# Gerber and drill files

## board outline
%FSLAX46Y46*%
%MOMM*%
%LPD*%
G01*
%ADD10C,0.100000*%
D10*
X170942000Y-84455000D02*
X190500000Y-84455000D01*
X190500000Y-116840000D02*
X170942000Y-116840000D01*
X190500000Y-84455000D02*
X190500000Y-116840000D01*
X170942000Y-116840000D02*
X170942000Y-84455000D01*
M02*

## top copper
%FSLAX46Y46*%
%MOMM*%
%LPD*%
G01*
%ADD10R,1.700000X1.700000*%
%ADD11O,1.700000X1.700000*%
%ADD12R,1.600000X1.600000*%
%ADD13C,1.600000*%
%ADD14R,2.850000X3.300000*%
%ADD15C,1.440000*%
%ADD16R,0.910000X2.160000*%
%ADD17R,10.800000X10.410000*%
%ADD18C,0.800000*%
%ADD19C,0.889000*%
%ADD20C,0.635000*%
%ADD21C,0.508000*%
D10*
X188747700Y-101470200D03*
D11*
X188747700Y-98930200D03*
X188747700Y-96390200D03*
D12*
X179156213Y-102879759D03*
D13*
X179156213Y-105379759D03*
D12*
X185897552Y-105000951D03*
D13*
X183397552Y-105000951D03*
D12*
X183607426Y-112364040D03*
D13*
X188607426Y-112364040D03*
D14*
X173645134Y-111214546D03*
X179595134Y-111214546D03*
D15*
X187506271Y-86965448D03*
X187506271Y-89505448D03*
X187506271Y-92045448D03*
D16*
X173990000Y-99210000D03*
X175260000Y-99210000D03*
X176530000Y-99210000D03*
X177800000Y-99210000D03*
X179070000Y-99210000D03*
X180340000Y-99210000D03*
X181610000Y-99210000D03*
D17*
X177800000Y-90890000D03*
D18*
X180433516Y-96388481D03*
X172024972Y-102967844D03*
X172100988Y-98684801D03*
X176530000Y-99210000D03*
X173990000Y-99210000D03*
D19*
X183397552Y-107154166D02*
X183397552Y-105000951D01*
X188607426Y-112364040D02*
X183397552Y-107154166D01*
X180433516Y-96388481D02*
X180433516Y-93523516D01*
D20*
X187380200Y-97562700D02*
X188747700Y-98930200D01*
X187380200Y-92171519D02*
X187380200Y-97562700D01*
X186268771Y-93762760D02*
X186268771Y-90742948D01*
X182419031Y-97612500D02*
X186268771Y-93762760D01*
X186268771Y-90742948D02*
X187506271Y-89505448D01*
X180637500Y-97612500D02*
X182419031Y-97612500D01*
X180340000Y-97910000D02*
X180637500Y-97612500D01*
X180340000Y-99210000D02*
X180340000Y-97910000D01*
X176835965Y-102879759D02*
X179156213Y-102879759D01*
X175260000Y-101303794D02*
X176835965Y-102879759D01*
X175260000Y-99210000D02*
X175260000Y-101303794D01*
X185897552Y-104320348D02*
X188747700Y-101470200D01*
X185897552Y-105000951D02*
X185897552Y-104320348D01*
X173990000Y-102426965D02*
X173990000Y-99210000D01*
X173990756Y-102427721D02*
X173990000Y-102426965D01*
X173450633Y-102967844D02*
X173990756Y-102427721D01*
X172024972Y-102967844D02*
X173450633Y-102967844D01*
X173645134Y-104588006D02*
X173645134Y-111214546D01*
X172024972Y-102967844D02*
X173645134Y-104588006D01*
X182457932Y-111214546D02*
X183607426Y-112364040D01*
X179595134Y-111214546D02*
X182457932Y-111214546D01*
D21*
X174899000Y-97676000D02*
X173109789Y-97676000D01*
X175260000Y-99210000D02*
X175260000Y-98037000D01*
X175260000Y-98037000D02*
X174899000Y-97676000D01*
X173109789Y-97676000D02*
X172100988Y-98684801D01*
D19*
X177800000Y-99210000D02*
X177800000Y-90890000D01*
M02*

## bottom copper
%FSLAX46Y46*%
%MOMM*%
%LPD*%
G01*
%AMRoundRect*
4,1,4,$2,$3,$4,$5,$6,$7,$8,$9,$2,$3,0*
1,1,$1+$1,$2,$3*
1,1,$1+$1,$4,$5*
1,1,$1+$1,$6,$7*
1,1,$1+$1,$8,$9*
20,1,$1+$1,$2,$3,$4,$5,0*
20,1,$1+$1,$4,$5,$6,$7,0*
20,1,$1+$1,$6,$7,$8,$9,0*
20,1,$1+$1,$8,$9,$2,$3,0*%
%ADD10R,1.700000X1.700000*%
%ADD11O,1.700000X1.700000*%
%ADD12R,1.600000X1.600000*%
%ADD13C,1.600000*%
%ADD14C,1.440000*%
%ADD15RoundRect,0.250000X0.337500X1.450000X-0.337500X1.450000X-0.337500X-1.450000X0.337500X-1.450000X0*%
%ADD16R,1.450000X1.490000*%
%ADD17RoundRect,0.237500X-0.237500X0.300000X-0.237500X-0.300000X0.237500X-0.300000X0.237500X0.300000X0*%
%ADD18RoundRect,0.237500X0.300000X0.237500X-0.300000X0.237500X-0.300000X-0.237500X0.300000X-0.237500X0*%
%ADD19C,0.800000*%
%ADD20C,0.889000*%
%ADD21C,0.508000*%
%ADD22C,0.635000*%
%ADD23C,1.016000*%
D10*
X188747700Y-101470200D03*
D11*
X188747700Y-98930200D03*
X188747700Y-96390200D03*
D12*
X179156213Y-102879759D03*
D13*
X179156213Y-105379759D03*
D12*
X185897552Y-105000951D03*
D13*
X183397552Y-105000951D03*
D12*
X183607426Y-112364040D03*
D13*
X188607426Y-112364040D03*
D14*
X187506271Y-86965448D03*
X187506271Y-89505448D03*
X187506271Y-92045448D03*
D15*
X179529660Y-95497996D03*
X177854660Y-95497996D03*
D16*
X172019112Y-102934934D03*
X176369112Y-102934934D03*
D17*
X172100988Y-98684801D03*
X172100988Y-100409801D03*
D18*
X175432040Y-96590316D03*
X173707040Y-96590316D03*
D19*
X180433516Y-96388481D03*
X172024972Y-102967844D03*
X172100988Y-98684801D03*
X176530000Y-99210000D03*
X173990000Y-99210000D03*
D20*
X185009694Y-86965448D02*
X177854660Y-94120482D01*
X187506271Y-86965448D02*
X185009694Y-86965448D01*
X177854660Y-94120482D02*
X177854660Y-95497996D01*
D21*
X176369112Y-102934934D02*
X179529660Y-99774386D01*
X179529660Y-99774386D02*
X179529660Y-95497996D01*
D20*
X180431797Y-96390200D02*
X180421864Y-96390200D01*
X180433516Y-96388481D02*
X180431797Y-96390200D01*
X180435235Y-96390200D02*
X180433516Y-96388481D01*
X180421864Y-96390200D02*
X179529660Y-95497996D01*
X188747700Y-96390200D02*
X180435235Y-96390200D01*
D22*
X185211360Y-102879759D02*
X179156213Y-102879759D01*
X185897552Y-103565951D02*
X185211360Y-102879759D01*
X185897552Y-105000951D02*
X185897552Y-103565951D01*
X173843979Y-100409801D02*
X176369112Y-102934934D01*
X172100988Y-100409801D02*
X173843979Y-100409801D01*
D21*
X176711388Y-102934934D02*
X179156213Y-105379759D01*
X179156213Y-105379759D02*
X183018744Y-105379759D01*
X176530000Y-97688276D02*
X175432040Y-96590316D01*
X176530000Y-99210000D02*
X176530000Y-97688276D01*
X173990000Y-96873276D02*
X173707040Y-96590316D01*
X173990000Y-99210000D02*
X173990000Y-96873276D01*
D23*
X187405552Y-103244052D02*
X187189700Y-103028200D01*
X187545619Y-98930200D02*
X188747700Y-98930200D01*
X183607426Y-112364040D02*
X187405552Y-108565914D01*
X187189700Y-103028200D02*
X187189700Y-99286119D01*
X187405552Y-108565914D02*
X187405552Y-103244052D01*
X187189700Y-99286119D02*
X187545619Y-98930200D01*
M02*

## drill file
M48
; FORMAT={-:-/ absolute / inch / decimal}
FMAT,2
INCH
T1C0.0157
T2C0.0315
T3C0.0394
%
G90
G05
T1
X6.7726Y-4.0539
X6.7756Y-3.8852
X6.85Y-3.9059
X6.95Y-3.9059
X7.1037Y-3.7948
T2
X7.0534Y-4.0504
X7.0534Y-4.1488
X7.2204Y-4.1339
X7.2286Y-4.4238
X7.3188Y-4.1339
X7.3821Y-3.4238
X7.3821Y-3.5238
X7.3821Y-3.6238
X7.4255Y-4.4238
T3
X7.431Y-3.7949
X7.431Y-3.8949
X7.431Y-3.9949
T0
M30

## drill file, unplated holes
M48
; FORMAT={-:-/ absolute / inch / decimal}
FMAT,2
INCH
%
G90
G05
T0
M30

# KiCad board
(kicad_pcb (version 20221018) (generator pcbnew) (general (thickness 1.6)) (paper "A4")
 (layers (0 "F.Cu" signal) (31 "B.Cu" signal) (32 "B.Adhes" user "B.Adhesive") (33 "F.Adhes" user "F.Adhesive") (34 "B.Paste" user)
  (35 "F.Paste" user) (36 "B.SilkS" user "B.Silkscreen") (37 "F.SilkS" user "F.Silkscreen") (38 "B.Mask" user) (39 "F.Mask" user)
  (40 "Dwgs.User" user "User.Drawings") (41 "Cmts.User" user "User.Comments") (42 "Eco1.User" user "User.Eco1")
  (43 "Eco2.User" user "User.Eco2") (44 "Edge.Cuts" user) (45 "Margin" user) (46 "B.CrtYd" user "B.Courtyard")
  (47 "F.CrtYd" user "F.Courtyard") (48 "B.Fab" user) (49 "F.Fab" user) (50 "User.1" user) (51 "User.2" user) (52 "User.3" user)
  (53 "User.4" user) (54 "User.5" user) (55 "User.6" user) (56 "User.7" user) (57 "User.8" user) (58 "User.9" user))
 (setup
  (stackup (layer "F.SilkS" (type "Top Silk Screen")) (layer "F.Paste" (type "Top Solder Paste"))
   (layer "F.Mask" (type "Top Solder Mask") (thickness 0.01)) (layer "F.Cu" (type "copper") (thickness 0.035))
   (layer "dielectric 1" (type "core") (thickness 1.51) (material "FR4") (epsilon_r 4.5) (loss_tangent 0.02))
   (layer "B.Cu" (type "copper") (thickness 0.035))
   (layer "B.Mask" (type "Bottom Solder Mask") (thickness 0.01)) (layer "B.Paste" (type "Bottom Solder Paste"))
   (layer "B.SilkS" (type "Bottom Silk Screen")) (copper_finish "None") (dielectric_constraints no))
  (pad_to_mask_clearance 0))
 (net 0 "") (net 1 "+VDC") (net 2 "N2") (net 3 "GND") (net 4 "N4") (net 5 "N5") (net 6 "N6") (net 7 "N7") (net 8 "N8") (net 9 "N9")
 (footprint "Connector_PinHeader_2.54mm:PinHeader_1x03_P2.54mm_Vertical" (layer "F.Cu") (at 188.7477 101.4702 180)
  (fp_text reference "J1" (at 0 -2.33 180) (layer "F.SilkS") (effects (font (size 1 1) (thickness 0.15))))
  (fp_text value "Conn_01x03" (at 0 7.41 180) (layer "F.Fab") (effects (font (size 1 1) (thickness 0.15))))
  (pad "1" thru_hole rect (at 0 0 180) (size 1.7 1.7) (drill 1) (layers "*.Cu" "*.Mask") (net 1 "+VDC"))
  (pad "2" thru_hole oval (at 0 2.54 180) (size 1.7 1.7) (drill 1) (layers "*.Cu" "*.Mask") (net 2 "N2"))
  (pad "3" thru_hole oval (at 0 5.08 180) (size 1.7 1.7) (drill 1) (layers "*.Cu" "*.Mask") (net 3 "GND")))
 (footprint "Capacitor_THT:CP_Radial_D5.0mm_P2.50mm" (layer "F.Cu") (at 179.156213 102.879759 -90)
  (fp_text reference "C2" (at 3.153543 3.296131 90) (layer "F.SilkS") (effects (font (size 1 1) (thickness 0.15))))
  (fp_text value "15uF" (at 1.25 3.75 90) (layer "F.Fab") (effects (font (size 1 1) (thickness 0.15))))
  (pad "1" thru_hole rect (at 0 0 270) (size 1.6 1.6) (drill 0.8) (layers "*.Cu" "*.Mask") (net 1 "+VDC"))
  (pad "2" thru_hole circle (at 2.5 0 270) (size 1.6 1.6) (drill 0.8) (layers "*.Cu" "*.Mask") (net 3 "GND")))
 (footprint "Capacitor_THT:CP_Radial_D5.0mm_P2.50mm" (layer "F.Cu") (at 185.897552 105.000951 180)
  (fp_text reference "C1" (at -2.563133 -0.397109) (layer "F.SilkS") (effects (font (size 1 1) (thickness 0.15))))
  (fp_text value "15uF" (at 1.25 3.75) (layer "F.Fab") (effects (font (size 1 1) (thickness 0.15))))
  (pad "1" thru_hole rect (at 0 0 180) (size 1.6 1.6) (drill 0.8) (layers "*.Cu" "*.Mask") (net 1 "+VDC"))
  (pad "2" thru_hole circle (at 2.5 0 180) (size 1.6 1.6) (drill 0.8) (layers "*.Cu" "*.Mask") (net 3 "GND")))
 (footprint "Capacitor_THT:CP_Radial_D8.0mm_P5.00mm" (layer "F.Cu") (at 183.607426 112.36404)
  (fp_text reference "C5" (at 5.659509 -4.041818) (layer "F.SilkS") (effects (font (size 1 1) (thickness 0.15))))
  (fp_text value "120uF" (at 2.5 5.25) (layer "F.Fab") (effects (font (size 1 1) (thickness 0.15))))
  (pad "1" thru_hole rect (at 0 0) (size 1.6 1.6) (drill 0.8) (layers "*.Cu" "*.Mask") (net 2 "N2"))
  (pad "2" thru_hole circle (at 5 0) (size 1.6 1.6) (drill 0.8) (layers "*.Cu" "*.Mask") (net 3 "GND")))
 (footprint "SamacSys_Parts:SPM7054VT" (layer "F.Cu") (at 176.620134 111.214546)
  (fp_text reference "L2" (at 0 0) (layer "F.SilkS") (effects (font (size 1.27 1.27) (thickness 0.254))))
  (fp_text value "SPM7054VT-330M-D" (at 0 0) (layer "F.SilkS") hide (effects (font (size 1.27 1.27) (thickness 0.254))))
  (pad "1" smd rect (at -2.975 0) (size 2.85 3.3) (layers "F.Cu" "F.Paste" "F.Mask") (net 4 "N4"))
  (pad "2" smd rect (at 2.975 0) (size 2.85 3.3) (layers "F.Cu" "F.Paste" "F.Mask") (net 2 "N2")))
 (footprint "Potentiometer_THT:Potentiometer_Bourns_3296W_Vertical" (layer "F.Cu") (at 187.506271 86.965448 90)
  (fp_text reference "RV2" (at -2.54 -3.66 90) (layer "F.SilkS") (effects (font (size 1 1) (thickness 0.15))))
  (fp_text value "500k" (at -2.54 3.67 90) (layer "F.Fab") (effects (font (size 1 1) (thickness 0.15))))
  (pad "1" thru_hole circle (at 0 0 90) (size 1.44 1.44) (drill 0.8) (layers "*.Cu" "*.Mask") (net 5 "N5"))
  (pad "2" thru_hole circle (at -2.54 0 90) (size 1.44 1.44) (drill 0.8) (layers "*.Cu" "*.Mask") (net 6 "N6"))
  (pad "3" thru_hole circle (at -5.08 0 90) (size 1.44 1.44) (drill 0.8) (layers "*.Cu" "*.Mask") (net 2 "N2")))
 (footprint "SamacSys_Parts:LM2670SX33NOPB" (layer "F.Cu") (at 177.8 91.44 -90)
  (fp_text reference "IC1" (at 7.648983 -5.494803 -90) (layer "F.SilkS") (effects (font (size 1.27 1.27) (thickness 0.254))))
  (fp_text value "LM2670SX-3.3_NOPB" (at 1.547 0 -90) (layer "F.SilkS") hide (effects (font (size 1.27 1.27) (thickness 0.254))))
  (pad "1" smd rect (at 7.77 3.81) (size 0.91 2.16) (layers "F.Cu" "F.Paste" "F.Mask") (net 4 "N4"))
  (pad "2" smd rect (at 7.77 2.54) (size 0.91 2.16) (layers "F.Cu" "F.Paste" "F.Mask") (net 1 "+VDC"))
  (pad "3" smd rect (at 7.77 1.27) (size 0.91 2.16) (layers "F.Cu" "F.Paste" "F.Mask") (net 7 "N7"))
  (pad "4" smd rect (at 7.77 0) (size 0.91 2.16) (layers "F.Cu" "F.Paste" "F.Mask") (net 3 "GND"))
  (pad "5" smd rect (at 7.77 -1.27) (size 0.91 2.16) (layers "F.Cu" "F.Paste" "F.Mask") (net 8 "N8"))
  (pad "6" smd rect (at 7.77 -2.54) (size 0.91 2.16) (layers "F.Cu" "F.Paste" "F.Mask") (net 6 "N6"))
  (pad "7" smd rect (at 7.77 -3.81) (size 0.91 2.16) (layers "F.Cu" "F.Paste" "F.Mask") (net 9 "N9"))
  (pad "8" smd rect (at -0.55 0 270) (size 10.41 10.8) (layers "F.Cu" "F.Paste" "F.Mask") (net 3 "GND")))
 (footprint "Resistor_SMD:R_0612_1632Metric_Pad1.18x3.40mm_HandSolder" (layer "B.Cu") (at 178.69216 95.497996 180)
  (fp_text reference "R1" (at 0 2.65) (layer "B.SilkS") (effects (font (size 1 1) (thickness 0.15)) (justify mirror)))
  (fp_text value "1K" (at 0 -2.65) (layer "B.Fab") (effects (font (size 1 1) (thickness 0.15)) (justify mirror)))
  (pad "1" smd roundrect (at -0.8375 0 180) (size 1.175 3.4) (layers "B.Cu" "B.Paste" "B.Mask") (roundrect_rratio 0.2127659574)
   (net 3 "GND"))
  (pad "2" smd roundrect (at 0.8375 0 180) (size 1.175 3.4) (layers "B.Cu" "B.Paste" "B.Mask") (roundrect_rratio 0.2127659574) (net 5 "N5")))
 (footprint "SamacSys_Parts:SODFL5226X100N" (layer "B.Cu") (at 174.194112 102.934934)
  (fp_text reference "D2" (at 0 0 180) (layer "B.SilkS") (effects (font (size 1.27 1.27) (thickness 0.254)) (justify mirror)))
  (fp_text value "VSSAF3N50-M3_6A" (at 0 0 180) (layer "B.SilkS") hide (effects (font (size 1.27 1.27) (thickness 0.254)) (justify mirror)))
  (pad "1" smd rect (at -2.175 0) (size 1.45 1.49) (layers "B.Cu" "B.Paste" "B.Mask") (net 4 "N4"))
  (pad "2" smd rect (at 2.175 0) (size 1.45 1.49) (layers "B.Cu" "B.Paste" "B.Mask") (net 3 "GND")))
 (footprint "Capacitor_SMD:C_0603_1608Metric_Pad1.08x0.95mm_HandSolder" (layer "B.Cu") (at 172.100988 99.547301 -90)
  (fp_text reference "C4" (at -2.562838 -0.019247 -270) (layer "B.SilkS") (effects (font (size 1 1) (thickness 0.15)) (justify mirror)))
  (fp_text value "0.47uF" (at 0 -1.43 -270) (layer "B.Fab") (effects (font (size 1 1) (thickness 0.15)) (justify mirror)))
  (pad "1" smd roundrect (at -0.8625 0 270) (size 1.075 0.95) (layers "B.Cu" "B.Paste" "B.Mask") (roundrect_rratio 0.25) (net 1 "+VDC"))
  (pad "2" smd roundrect (at 0.8625 0 270) (size 1.075 0.95) (layers "B.Cu" "B.Paste" "B.Mask") (roundrect_rratio 0.25) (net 3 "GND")))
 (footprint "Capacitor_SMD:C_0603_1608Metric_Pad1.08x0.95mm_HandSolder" (layer "B.Cu") (at 174.56954 96.590316 180)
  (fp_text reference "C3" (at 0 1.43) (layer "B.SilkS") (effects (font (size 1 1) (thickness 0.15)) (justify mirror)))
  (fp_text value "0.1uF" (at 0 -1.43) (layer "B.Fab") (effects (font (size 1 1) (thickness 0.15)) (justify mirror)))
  (pad "1" smd roundrect (at -0.8625 0 180) (size 1.075 0.95) (layers "B.Cu" "B.Paste" "B.Mask") (roundrect_rratio 0.25) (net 7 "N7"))
  (pad "2" smd roundrect (at 0.8625 0 180) (size 1.075 0.95) (layers "B.Cu" "B.Paste" "B.Mask") (roundrect_rratio 0.25) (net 4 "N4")))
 (gr_line (start 170.942 84.455) (end 190.5 84.455) (stroke (width 0.1) (type solid)) (layer "Edge.Cuts"))
 (gr_line (start 190.5 116.84) (end 170.942 116.84) (stroke (width 0.1) (type default)) (layer "Edge.Cuts"))
 (gr_line (start 190.5 84.455) (end 190.5 116.84) (stroke (width 0.1) (type default)) (layer "Edge.Cuts"))
 (gr_line (start 170.942 116.84) (end 170.942 84.455) (stroke (width 0.1) (type solid)) (layer "Edge.Cuts"))
 (segment (start 175.26 99.21) (end 175.26 101.303794) (width 0.635) (layer "F.Cu") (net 1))
 (segment (start 174.899 97.676) (end 173.109789 97.676) (width 0.508) (layer "F.Cu") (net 1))
 (segment (start 175.26 101.303794) (end 176.835965 102.879759) (width 0.635) (layer "F.Cu") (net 1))
 (segment (start 185.897552 105.000951) (end 185.897552 104.320348) (width 0.635) (layer "F.Cu") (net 1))
 (segment (start 175.26 99.21) (end 175.26 98.037) (width 0.508) (layer "F.Cu") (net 1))
 (segment (start 175.26 98.037) (end 174.899 97.676) (width 0.508) (layer "F.Cu") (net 1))
 (segment (start 176.835965 102.879759) (end 179.156213 102.879759) (width 0.635) (layer "F.Cu") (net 1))
 (segment (start 185.897552 104.320348) (end 188.7477 101.4702) (width 0.635) (layer "F.Cu") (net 1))
 (segment (start 173.109789 97.676) (end 172.100988 98.684801) (width 0.508) (layer "F.Cu") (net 1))
 (via (at 172.100988 98.684801) (size 0.8) (drill 0.4) (layers "F.Cu" "B.Cu") (free) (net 1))
 (segment (start 185.897552 105.000951) (end 185.897552 103.565951) (width 0.635) (layer "B.Cu") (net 1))
 (segment (start 185.21136 102.879759) (end 179.156213 102.879759) (width 0.635) (layer "B.Cu") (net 1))
 (segment (start 185.897552 103.565951) (end 185.21136 102.879759) (width 0.635) (layer "B.Cu") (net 1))
 (segment (start 180.433516 96.388481) (end 180.433516 93.523516) (width 0.889) (layer "F.Cu") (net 3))
 (segment (start 177.8 99.21) (end 177.8 90.89) (width 0.889) (layer "F.Cu") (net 3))
 (segment (start 183.397552 107.154166) (end 183.397552 105.000951) (width 0.889) (layer "F.Cu") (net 3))
 (segment (start 188.607426 112.36404) (end 183.397552 107.154166) (width 0.889) (layer "F.Cu") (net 3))
 (via (at 180.433516 96.388481) (size 0.8) (drill 0.4) (layers "F.Cu" "B.Cu") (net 3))
 (segment (start 173.843979 100.409801) (end 176.369112 102.934934) (width 0.635) (layer "B.Cu") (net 3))
 (segment (start 180.431797 96.3902) (end 180.421864 96.3902) (width 0.889) (layer "B.Cu") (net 3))
 (segment (start 176.369112 102.934934) (end 179.52966 99.774386) (width 0.508) (layer "B.Cu") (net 3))
 (segment (start 180.421864 96.3902) (end 179.52966 95.497996) (width 0.889) (layer "B.Cu") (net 3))
 (segment (start 176.711388 102.934934) (end 179.156213 105.379759) (width 0.508) (layer "B.Cu") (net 3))
 (segment (start 179.52966 99.774386) (end 179.52966 95.497996) (width 0.508) (layer "B.Cu") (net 3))
 (segment (start 179.156213 105.379759) (end 183.018744 105.379759) (width 0.508) (layer "B.Cu") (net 3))
 (segment (start 188.7477 96.3902) (end 180.435235 96.3902) (width 0.889) (layer "B.Cu") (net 3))
 (segment (start 180.435235 96.3902) (end 180.433516 96.388481) (width 0.889) (layer "B.Cu") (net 3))
 (segment (start 180.433516 96.388481) (end 180.431797 96.3902) (width 0.889) (layer "B.Cu") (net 3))
 (segment (start 172.100988 100.409801) (end 173.843979 100.409801) (width 0.635) (layer "B.Cu") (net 3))
 (via (at 176.53 99.21) (size 0.8) (drill 0.4) (layers "F.Cu" "B.Cu") (free) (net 7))
 (segment (start 176.53 97.688276) (end 175.43204 96.590316) (width 0.508) (layer "B.Cu") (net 7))
 (segment (start 176.53 99.21) (end 176.53 97.688276) (width 0.508) (layer "B.Cu") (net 7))
 (segment (start 173.990756 102.427721) (end 173.99 102.426965) (width 0.635) (layer "F.Cu") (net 4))
 (segment (start 173.450633 102.967844) (end 173.990756 102.427721) (width 0.635) (layer "F.Cu") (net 4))
 (segment (start 173.645134 104.588006) (end 173.645134 111.214546) (width 0.635) (layer "F.Cu") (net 4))
 (segment (start 172.024972 102.967844) (end 173.450633 102.967844) (width 0.635) (layer "F.Cu") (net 4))
 (segment (start 173.99 102.426965) (end 173.99 99.21) (width 0.635) (layer "F.Cu") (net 4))
 (segment (start 172.024972 102.967844) (end 173.645134 104.588006) (width 0.635) (layer "F.Cu") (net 4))
 (via (at 172.024972 102.967844) (size 0.8) (drill 0.4) (layers "F.Cu" "B.Cu") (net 4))
 (via (at 173.99 99.21) (size 0.8) (drill 0.4) (layers "F.Cu" "B.Cu") (free) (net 4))
 (segment (start 173.99 96.873276) (end 173.70704 96.590316) (width 0.508) (layer "B.Cu") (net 4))
 (segment (start 173.99 99.21) (end 173.99 96.873276) (width 0.508) (layer "B.Cu") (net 4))
 (segment (start 182.457932 111.214546) (end 183.607426 112.36404) (width 0.635) (layer "F.Cu") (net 2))
 (segment (start 187.3802 92.171519) (end 187.3802 97.5627) (width 0.635) (layer "F.Cu") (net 2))
 (segment (start 179.595134 111.214546) (end 182.457932 111.214546) (width 0.635) (layer "F.Cu") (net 2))
 (segment (start 187.3802 97.5627) (end 188.7477 98.9302) (width 0.635) (layer "F.Cu") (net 2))
 (segment (start 187.405552 103.244052) (end 187.1897 103.0282) (width 1.016) (layer "B.Cu") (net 2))
 (segment (start 187.545619 98.9302) (end 188.7477 98.9302) (width 1.016) (layer "B.Cu") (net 2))
 (segment (start 183.607426 112.36404) (end 187.405552 108.565914) (width 1.016) (layer "B.Cu") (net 2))
 (segment (start 187.1897 103.0282) (end 187.1897 99.286119) (width 1.016) (layer "B.Cu") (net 2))
 (segment (start 187.405552 108.565914) (end 187.405552 103.244052) (width 1.016) (layer "B.Cu") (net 2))
 (segment (start 187.1897 99.286119) (end 187.545619 98.9302) (width 1.016) (layer "B.Cu") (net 2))
 (segment (start 182.419031 97.6125) (end 186.268771 93.76276) (width 0.635) (layer "F.Cu") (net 6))
 (segment (start 180.6375 97.6125) (end 182.419031 97.6125) (width 0.635) (layer "F.Cu") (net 6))
 (segment (start 186.268771 90.742948) (end 187.506271 89.505448) (width 0.635) (layer "F.Cu") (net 6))
 (segment (start 186.268771 93.76276) (end 186.268771 90.742948) (width 0.635) (layer "F.Cu") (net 6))
 (segment (start 180.34 97.91) (end 180.6375 97.6125) (width 0.635) (layer "F.Cu") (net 6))
 (segment (start 180.34 99.21) (end 180.34 97.91) (width 0.635) (layer "F.Cu") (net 6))
 (segment (start 177.85466 94.120482) (end 177.85466 95.497996) (width 0.889) (layer "B.Cu") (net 5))
 (segment (start 185.009694 86.965448) (end 177.85466 94.120482) (width 0.889) (layer "B.Cu") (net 5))
 (segment (start 187.506271 86.965448) (end 185.009694 86.965448) (width 0.889) (layer "B.Cu") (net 5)))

